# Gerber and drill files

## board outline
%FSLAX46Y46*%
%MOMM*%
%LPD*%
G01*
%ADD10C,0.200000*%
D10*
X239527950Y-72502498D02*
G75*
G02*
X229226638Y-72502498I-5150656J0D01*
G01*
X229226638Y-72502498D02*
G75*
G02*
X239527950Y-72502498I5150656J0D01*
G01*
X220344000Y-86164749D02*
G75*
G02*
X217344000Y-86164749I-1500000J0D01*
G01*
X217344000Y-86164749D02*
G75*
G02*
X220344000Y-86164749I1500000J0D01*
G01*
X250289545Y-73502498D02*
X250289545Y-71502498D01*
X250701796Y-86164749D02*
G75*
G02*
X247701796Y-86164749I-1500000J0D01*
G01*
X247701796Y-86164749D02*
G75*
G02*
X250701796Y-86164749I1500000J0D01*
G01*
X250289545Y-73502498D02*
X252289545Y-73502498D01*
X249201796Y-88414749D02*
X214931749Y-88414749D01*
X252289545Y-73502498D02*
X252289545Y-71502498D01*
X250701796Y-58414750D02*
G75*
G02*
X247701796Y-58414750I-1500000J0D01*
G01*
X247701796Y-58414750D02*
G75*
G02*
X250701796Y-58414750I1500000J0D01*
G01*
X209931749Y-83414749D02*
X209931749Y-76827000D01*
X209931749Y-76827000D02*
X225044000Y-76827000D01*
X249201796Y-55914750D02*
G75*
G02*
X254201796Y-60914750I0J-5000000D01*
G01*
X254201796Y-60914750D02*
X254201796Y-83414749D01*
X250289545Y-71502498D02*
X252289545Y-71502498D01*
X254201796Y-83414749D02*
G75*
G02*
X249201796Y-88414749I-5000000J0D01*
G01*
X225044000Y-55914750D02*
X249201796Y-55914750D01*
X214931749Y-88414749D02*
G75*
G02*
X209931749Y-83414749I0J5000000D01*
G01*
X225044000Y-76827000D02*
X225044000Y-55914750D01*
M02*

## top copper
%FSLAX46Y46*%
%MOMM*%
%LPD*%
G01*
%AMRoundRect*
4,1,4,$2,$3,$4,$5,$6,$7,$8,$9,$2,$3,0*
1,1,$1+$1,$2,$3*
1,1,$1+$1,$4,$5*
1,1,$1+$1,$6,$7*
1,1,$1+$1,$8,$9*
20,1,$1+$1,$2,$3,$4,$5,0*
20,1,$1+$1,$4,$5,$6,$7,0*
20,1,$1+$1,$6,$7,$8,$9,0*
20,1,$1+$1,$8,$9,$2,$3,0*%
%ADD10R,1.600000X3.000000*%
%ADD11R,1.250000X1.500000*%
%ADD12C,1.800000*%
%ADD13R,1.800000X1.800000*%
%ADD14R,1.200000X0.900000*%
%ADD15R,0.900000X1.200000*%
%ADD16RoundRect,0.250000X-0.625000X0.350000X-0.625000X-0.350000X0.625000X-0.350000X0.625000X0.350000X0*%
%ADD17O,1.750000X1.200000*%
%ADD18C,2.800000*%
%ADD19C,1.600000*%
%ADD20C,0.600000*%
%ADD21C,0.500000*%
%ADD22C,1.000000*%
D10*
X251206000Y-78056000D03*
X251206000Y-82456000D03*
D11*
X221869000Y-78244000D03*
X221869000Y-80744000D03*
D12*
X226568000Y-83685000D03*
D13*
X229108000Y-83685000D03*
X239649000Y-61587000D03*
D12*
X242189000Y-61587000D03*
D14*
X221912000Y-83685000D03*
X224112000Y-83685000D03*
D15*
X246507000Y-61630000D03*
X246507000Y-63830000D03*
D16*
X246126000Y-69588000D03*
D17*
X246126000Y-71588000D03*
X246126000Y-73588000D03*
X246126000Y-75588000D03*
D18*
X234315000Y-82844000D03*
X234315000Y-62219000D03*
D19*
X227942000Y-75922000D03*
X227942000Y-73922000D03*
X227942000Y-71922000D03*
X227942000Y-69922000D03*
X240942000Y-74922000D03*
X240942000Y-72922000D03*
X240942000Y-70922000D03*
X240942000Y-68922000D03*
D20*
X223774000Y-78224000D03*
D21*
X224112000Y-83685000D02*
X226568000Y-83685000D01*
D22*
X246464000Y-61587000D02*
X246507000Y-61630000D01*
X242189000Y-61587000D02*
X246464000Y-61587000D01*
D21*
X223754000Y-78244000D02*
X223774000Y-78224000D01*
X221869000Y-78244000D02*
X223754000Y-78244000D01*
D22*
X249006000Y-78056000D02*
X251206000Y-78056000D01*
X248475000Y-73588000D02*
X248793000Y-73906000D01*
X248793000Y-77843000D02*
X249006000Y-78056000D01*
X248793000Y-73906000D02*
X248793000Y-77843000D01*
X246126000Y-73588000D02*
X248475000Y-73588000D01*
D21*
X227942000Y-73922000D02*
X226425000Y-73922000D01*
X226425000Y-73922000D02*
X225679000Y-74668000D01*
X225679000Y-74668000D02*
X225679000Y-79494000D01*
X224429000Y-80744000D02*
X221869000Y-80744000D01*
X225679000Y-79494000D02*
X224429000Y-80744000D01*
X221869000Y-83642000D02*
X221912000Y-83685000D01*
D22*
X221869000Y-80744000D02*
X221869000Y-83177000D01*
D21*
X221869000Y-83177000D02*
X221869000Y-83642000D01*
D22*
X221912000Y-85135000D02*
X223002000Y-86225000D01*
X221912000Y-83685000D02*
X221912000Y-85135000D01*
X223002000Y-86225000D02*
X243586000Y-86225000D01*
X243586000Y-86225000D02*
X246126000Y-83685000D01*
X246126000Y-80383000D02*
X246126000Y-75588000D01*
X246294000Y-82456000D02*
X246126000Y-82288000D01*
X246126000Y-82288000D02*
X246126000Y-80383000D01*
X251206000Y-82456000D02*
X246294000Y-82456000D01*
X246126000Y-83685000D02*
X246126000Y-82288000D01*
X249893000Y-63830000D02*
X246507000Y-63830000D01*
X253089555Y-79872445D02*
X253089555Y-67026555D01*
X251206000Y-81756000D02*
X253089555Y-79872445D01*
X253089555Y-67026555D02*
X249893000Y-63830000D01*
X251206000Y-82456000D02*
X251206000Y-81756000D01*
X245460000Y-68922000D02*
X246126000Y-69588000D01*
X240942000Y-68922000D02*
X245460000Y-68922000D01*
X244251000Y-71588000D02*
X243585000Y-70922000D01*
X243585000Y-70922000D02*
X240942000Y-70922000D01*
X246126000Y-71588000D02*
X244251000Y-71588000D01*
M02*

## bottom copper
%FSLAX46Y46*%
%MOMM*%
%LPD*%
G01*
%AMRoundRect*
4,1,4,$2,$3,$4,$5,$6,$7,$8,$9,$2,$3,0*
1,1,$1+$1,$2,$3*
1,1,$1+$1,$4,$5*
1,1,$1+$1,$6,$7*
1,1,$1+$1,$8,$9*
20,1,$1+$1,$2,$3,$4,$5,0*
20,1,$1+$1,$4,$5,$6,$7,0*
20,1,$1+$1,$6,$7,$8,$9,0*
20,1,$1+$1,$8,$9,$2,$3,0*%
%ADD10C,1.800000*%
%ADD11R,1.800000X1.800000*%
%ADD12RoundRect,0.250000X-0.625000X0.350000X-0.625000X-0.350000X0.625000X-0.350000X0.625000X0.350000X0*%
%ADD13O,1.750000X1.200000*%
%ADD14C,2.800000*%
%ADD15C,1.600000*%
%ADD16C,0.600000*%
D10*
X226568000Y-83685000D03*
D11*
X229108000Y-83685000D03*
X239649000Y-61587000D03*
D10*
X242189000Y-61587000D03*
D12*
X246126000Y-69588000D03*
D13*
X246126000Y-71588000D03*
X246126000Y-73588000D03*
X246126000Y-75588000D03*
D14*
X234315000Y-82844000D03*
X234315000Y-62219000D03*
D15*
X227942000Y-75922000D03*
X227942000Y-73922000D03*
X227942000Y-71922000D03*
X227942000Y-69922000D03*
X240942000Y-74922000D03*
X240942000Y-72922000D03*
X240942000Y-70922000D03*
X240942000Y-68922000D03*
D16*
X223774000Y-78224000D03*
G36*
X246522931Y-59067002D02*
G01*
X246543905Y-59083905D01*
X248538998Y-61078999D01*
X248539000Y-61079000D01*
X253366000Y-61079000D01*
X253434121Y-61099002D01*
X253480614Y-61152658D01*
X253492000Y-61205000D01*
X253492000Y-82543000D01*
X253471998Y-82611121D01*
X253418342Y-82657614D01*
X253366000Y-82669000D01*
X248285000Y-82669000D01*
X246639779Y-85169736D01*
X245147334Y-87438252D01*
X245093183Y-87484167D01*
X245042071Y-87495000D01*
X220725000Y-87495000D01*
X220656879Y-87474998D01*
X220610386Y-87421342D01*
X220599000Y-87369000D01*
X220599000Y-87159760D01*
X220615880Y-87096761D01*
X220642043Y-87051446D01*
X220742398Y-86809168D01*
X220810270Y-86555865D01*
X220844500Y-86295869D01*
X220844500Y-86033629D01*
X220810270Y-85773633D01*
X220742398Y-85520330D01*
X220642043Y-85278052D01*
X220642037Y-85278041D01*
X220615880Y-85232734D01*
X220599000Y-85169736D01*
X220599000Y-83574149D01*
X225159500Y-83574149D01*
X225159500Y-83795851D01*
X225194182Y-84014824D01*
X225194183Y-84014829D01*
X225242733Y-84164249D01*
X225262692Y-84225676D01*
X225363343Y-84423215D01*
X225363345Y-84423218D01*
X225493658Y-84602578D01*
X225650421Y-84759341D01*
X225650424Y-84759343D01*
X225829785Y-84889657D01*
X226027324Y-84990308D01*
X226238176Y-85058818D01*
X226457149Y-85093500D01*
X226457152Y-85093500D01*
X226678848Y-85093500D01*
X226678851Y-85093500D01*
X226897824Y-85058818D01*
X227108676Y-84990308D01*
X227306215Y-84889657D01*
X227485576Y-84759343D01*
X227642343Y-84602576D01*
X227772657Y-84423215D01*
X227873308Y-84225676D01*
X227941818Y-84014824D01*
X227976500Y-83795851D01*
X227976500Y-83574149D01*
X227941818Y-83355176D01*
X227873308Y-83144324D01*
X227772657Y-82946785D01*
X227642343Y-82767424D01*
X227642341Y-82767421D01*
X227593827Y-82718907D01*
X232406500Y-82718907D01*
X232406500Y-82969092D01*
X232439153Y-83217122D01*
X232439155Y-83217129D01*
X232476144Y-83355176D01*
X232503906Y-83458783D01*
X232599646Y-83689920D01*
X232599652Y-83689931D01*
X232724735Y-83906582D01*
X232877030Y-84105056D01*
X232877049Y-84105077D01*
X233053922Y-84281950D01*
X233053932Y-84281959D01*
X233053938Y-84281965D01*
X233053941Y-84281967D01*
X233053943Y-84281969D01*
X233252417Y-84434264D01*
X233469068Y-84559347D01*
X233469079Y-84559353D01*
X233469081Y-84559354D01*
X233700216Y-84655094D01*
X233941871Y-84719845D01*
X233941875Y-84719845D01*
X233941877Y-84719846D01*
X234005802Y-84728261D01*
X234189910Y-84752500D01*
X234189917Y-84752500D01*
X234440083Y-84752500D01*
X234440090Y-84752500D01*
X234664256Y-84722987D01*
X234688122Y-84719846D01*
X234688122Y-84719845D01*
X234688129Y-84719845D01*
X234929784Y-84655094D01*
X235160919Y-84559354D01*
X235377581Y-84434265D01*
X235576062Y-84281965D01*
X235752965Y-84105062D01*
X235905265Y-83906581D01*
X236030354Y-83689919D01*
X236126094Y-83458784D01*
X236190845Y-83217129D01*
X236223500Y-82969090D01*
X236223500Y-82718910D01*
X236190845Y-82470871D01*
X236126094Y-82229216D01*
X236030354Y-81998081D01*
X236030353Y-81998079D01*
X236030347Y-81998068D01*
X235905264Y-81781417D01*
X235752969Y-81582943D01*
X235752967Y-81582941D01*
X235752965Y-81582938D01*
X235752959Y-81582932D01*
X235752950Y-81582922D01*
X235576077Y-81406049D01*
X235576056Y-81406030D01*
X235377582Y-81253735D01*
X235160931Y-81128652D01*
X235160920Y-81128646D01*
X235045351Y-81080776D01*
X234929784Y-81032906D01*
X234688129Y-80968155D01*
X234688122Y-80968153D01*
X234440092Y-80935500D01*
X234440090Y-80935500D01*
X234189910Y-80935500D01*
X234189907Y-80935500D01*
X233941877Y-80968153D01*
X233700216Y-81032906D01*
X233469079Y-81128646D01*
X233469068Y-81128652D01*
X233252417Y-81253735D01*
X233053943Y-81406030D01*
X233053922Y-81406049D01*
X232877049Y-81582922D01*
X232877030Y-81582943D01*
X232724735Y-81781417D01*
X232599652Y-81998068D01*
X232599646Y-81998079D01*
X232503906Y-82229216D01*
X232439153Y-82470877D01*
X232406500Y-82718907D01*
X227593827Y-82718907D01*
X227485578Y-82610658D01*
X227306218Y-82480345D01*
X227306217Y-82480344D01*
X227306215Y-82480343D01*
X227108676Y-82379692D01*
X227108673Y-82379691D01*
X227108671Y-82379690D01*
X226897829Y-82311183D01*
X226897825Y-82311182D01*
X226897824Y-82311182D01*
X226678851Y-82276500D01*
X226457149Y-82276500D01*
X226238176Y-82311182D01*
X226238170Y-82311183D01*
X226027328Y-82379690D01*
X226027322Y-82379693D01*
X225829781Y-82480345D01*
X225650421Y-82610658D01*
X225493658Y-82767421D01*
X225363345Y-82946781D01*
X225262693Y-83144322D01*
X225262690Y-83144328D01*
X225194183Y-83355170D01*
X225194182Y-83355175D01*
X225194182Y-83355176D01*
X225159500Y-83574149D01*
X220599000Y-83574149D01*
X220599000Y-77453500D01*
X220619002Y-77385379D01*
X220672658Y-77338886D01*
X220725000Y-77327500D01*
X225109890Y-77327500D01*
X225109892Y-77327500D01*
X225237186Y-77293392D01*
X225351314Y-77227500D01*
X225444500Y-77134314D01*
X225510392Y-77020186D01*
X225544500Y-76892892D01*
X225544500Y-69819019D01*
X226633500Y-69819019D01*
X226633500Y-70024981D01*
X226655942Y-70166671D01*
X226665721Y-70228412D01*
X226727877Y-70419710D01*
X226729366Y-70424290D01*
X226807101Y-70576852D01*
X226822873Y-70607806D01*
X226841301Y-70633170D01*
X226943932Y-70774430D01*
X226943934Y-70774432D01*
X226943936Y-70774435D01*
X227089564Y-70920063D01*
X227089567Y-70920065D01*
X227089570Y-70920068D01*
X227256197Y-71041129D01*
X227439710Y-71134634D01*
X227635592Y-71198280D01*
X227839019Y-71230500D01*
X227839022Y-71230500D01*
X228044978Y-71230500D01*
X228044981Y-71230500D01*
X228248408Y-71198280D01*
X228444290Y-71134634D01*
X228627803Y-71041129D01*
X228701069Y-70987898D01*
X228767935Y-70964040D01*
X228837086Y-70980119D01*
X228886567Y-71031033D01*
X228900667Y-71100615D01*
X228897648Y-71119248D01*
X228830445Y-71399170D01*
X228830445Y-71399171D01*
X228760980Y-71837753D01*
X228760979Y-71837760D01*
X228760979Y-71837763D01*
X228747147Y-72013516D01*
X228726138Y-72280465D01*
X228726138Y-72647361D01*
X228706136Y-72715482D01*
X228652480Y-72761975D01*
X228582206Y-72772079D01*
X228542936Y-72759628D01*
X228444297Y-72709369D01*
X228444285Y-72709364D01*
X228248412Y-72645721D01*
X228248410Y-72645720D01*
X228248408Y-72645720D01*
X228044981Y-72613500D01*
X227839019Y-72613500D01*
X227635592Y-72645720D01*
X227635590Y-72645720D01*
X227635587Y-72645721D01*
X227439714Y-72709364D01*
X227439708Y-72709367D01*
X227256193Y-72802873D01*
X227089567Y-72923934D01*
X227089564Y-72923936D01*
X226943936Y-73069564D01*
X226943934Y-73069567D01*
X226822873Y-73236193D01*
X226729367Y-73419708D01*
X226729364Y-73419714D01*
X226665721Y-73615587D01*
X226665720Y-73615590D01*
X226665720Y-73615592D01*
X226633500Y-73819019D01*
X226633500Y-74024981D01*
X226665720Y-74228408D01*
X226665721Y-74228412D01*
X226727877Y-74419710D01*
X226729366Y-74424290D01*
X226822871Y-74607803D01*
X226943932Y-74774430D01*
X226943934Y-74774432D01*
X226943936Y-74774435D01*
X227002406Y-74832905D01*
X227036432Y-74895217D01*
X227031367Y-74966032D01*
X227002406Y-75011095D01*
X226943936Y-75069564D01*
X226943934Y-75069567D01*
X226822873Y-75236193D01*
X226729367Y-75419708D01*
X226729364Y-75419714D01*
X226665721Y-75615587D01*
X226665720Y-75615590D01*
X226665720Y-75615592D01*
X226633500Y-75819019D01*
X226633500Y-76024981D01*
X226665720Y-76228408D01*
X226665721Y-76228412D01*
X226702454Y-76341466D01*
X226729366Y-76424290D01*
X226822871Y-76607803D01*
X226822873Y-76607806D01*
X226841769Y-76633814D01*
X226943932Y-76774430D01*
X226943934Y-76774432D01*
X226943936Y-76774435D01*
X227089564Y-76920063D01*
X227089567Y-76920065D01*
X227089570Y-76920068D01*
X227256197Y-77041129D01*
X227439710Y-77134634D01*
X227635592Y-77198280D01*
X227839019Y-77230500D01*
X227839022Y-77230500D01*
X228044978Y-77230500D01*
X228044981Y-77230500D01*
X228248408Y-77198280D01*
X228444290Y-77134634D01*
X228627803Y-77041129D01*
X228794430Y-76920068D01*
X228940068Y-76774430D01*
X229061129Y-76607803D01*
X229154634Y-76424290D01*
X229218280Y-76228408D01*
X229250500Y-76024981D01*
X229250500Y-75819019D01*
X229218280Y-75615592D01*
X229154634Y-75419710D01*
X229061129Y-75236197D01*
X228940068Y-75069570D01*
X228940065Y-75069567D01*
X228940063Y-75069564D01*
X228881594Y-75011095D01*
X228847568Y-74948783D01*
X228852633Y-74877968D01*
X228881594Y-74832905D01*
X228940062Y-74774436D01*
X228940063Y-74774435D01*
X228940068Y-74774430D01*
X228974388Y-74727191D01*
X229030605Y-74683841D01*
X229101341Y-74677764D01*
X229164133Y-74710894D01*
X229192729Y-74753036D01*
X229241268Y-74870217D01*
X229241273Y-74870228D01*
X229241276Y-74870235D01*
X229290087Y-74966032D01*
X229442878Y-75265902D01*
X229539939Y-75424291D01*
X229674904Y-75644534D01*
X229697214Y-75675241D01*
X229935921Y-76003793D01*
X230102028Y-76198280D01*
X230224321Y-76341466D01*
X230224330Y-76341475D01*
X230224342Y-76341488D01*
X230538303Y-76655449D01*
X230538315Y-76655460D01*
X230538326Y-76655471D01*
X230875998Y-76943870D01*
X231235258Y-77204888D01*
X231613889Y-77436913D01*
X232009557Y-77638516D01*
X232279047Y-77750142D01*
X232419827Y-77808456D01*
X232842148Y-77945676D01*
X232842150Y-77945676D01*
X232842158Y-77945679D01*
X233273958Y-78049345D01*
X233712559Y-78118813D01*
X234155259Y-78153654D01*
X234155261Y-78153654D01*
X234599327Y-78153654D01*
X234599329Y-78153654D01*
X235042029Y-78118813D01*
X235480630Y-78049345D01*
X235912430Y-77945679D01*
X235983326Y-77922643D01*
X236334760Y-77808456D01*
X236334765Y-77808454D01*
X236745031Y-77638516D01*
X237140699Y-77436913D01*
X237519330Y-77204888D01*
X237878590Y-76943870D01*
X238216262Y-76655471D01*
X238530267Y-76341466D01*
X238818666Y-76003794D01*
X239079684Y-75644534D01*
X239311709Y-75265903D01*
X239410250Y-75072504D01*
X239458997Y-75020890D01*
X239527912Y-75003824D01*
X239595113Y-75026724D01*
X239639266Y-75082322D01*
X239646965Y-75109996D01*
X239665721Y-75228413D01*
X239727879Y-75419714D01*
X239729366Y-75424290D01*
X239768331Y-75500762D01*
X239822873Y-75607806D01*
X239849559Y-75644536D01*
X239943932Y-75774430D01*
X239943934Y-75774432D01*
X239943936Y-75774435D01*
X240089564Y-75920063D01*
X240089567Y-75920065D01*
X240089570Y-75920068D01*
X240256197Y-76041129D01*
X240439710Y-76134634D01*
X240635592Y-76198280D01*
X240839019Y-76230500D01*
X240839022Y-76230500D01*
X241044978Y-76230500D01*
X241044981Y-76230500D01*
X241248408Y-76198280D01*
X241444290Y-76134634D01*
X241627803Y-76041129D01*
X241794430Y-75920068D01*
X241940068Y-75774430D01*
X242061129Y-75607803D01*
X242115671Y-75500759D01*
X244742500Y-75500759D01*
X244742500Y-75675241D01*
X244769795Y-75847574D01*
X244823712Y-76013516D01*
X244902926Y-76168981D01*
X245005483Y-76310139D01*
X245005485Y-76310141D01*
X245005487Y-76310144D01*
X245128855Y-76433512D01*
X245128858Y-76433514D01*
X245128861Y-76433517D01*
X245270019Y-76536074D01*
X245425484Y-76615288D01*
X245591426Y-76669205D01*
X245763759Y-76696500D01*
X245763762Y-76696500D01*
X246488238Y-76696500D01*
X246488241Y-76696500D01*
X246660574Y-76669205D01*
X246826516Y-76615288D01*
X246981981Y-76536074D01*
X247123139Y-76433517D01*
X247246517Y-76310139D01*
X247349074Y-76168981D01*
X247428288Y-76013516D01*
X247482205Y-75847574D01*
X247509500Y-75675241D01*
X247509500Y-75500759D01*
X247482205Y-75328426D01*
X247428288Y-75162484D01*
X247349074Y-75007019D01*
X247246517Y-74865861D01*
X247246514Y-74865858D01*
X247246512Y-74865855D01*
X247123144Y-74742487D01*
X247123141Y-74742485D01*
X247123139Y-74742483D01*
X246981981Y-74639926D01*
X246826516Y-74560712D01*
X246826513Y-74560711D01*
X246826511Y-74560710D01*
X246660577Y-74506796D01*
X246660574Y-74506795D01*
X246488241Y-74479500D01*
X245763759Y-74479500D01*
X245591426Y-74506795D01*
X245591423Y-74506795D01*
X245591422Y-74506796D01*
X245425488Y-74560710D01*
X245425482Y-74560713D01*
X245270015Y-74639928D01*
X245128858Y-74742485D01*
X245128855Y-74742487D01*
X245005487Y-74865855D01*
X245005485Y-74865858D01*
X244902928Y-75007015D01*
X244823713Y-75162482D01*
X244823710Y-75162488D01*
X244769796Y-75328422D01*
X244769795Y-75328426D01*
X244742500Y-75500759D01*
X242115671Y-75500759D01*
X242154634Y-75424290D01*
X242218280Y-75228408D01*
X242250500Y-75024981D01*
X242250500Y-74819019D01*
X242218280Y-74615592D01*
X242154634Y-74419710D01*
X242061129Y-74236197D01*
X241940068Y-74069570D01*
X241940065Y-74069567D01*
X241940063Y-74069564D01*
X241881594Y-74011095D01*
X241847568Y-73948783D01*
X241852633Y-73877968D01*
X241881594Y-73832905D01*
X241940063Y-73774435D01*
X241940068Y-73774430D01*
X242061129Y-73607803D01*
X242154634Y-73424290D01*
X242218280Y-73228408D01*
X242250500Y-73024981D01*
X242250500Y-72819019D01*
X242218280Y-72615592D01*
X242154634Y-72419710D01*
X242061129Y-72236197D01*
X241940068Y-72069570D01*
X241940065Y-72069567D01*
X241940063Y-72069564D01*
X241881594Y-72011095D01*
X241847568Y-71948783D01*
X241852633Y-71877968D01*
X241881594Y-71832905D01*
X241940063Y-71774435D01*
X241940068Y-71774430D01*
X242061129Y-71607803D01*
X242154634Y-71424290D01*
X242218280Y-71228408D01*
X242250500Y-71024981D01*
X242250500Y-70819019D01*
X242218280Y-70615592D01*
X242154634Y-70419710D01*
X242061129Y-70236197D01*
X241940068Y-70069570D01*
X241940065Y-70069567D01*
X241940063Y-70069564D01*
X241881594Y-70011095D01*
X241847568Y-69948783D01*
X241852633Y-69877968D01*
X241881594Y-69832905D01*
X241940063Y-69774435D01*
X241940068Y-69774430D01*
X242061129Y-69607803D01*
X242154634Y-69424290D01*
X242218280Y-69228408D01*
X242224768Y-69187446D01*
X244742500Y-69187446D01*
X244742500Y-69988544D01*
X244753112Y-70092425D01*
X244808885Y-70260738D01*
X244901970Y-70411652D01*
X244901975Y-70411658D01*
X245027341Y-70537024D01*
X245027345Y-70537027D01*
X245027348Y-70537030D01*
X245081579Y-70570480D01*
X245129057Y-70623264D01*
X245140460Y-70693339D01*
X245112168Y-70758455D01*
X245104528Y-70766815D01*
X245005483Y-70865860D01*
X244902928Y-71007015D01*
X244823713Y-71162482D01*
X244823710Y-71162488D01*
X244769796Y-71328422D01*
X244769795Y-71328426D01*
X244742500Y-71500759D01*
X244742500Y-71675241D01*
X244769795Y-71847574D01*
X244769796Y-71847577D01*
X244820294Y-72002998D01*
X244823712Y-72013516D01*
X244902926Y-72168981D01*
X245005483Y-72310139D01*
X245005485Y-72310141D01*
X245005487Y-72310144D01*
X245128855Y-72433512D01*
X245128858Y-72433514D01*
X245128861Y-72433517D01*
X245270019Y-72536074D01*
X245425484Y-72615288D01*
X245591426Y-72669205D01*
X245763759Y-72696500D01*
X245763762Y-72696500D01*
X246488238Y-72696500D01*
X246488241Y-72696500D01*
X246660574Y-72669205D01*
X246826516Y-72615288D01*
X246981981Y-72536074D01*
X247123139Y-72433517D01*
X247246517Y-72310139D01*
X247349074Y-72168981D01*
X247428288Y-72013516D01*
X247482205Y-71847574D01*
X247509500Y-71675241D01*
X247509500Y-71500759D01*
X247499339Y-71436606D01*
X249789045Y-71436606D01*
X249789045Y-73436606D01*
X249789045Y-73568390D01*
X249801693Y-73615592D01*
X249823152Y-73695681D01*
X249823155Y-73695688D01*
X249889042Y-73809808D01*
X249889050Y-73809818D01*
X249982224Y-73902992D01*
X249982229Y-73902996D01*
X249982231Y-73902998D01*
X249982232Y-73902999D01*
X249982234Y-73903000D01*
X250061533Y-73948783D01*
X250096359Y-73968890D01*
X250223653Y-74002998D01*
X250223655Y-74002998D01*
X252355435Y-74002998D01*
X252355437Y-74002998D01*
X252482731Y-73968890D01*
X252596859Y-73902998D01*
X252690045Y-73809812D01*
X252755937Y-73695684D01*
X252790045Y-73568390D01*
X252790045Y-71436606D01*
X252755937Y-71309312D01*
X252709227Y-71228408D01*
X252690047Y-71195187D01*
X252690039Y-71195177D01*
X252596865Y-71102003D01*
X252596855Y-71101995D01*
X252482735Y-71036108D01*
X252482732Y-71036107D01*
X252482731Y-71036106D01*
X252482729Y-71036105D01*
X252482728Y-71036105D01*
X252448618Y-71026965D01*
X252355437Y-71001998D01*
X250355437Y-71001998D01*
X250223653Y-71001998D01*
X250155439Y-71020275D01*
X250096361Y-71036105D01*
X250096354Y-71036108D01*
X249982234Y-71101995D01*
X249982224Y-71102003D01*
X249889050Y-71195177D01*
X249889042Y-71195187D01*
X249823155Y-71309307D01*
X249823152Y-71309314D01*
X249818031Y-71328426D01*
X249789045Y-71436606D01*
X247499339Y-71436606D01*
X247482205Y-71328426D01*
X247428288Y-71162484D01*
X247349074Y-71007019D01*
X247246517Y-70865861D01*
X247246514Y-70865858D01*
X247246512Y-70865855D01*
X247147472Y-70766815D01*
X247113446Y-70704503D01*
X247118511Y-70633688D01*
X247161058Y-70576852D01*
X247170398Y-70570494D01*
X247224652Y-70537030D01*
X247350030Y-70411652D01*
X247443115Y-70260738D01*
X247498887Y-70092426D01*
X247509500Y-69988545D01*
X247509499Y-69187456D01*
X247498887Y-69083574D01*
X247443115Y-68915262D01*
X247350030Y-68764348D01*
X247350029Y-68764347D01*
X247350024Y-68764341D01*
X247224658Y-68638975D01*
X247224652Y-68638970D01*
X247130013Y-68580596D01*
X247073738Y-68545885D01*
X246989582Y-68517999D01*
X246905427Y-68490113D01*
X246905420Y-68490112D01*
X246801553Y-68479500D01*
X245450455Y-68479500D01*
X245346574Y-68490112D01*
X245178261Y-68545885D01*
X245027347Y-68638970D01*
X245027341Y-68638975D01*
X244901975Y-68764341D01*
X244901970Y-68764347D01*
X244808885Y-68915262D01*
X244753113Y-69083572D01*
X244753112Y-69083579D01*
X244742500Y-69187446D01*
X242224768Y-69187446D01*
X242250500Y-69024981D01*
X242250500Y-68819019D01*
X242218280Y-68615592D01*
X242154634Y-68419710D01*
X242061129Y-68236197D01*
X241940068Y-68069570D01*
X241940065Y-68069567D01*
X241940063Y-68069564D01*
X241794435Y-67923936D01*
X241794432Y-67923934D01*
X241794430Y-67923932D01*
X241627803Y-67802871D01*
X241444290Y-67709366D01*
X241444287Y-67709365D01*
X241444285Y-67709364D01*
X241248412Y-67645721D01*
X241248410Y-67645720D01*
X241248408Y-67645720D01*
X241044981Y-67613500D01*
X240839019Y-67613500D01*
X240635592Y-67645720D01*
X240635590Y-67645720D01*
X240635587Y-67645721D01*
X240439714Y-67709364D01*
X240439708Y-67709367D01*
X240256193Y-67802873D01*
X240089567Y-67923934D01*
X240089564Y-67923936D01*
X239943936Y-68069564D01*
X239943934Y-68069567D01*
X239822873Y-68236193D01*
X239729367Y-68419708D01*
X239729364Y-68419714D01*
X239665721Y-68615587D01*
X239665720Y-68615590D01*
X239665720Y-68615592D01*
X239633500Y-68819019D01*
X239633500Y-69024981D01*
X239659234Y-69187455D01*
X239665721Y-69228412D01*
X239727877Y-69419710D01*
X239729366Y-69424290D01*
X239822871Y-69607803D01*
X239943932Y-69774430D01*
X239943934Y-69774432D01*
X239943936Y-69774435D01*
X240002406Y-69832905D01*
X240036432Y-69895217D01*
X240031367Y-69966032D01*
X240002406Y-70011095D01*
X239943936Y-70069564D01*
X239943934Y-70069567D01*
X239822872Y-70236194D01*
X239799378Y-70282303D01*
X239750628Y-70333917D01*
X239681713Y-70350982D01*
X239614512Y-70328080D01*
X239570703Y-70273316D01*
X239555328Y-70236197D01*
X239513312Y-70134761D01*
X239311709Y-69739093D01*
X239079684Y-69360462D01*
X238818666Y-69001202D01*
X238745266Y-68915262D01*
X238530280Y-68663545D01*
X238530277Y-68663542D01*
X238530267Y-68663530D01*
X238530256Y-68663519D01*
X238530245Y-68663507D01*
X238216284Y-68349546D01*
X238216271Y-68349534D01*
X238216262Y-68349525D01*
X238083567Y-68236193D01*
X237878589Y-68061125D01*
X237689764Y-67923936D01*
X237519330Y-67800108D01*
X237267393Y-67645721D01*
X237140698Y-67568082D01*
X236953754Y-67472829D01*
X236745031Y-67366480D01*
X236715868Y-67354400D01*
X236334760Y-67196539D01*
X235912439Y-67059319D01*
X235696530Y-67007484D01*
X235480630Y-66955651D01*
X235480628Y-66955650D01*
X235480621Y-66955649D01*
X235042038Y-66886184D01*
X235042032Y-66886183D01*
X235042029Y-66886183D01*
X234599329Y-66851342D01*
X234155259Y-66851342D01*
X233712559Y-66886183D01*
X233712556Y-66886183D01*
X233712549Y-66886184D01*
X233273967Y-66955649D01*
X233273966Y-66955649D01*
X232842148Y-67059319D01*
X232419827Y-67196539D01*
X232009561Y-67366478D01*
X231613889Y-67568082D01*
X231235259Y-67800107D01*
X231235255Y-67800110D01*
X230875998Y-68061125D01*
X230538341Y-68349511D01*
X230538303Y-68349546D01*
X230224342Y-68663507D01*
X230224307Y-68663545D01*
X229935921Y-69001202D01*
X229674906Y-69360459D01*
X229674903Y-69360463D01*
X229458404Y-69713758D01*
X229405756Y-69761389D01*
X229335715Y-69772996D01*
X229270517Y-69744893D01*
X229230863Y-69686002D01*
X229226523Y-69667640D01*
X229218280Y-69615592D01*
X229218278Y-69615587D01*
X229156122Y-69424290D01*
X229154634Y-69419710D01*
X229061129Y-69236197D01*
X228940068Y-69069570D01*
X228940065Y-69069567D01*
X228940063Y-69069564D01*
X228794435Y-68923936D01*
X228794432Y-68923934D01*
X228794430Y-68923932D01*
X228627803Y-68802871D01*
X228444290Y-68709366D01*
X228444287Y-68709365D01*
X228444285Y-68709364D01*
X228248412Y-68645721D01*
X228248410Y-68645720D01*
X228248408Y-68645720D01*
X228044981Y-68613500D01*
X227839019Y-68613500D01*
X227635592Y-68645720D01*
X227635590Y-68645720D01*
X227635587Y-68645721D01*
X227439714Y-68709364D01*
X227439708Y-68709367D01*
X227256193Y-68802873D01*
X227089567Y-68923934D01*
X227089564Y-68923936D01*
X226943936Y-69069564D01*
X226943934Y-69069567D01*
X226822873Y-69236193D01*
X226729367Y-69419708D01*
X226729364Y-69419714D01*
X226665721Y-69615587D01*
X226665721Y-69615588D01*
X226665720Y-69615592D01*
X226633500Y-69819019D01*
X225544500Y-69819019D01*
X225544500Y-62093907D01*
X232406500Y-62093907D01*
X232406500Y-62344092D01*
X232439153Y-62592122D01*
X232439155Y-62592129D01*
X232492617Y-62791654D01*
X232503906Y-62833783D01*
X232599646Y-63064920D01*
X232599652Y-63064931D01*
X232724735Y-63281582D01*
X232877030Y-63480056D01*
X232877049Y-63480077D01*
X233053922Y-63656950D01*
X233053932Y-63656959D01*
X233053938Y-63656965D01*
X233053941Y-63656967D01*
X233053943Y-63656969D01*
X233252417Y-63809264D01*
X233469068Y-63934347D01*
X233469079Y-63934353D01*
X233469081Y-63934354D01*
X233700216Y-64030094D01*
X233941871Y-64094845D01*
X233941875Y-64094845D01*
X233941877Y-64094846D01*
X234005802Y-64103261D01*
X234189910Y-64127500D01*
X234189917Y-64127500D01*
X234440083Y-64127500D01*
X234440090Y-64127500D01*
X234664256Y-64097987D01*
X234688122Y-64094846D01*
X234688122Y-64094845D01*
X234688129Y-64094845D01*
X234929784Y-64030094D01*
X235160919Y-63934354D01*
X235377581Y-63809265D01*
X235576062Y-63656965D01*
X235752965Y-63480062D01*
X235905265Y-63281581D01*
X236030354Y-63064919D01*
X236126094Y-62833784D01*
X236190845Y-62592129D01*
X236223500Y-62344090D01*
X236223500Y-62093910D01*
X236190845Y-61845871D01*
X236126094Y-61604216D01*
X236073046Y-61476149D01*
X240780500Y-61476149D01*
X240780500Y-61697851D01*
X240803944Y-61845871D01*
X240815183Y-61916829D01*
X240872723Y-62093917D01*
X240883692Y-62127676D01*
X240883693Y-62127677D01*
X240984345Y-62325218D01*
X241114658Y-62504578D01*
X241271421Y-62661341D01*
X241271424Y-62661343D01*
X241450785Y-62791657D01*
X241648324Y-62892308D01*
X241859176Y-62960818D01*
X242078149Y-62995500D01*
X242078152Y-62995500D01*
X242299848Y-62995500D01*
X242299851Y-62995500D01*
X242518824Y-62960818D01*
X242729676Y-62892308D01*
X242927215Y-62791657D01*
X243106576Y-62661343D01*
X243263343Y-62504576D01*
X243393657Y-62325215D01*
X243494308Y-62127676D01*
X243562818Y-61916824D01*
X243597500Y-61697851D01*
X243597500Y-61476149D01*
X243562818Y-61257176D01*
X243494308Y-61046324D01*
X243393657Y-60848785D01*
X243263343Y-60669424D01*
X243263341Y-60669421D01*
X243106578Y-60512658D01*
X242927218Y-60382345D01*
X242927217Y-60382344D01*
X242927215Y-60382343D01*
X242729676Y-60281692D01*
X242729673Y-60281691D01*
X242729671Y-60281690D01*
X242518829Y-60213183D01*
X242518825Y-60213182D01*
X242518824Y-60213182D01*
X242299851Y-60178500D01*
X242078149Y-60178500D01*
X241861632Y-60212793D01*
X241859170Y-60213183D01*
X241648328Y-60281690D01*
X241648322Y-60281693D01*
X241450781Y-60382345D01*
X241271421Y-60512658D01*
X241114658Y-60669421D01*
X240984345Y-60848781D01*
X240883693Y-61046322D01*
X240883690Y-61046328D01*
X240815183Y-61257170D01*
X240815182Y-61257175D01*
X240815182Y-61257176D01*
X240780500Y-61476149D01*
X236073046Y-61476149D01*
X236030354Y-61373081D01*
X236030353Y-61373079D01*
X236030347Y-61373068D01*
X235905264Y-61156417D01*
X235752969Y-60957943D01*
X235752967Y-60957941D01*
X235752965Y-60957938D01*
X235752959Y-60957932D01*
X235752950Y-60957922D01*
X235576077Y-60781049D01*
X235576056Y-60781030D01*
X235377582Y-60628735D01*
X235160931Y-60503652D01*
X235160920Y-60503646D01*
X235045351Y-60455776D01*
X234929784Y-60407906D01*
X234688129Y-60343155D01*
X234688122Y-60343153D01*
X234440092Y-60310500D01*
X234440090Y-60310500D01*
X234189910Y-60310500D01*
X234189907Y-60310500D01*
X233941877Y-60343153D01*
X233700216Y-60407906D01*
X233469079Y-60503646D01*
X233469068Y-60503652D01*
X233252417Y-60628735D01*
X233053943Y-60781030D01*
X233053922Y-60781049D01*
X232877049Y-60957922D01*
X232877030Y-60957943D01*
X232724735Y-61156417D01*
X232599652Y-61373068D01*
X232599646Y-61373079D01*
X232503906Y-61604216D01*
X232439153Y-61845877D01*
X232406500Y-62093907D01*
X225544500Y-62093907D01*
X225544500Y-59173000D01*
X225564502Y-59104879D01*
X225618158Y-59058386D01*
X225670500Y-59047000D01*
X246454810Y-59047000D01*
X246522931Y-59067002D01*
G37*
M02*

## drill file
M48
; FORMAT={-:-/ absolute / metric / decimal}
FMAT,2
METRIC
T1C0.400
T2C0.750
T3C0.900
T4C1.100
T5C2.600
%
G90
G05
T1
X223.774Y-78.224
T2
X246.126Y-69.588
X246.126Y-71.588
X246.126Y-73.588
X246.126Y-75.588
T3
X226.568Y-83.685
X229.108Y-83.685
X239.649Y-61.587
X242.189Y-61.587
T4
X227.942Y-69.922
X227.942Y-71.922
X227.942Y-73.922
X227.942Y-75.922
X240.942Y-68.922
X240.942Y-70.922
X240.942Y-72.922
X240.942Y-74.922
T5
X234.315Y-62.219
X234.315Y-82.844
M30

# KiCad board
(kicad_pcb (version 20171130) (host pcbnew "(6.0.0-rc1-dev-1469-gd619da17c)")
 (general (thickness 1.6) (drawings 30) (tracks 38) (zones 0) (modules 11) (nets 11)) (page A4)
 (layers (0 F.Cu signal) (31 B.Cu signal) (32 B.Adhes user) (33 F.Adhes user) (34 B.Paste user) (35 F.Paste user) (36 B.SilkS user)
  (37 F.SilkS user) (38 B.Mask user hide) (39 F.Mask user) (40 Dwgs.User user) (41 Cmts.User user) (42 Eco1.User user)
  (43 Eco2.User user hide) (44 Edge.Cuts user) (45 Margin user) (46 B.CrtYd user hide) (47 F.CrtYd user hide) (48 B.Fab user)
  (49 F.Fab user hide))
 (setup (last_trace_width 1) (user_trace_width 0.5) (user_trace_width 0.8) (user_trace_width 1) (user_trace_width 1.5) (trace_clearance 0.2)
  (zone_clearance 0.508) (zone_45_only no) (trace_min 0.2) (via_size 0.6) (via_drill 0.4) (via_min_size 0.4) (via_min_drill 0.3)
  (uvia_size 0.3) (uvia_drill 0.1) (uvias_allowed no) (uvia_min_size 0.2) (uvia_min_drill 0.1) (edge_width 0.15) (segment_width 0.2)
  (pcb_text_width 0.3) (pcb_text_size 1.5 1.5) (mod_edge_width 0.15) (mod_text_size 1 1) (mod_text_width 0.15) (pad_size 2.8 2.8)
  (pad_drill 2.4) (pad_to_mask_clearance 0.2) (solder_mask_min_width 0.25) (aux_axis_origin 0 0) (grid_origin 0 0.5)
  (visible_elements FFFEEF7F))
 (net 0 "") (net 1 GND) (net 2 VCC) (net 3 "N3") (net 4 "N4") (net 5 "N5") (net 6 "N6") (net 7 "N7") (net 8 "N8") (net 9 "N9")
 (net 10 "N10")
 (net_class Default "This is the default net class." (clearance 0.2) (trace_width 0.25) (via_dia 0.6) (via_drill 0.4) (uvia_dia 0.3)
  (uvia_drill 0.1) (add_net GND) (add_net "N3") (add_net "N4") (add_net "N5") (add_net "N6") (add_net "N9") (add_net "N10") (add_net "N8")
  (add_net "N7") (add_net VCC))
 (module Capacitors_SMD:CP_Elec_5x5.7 (layer F.Cu) (at 251.206 80.256 90)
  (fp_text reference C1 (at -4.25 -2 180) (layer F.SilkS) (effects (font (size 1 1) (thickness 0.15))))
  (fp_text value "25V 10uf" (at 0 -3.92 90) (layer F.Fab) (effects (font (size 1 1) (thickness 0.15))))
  (pad 2 smd rect (at 2.2 0 270) (size 3 1.6) (layers F.Cu F.Paste F.Mask) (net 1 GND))
  (pad 1 smd rect (at -2.2 0 270) (size 3 1.6) (layers F.Cu F.Paste F.Mask) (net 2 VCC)))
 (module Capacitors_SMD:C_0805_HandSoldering (layer F.Cu) (at 221.869 79.494 90)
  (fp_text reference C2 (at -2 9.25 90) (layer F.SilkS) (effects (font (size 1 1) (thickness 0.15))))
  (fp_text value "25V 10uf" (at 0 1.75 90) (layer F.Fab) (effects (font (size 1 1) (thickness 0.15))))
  (pad 2 smd rect (at 1.25 0 90) (size 1.5 1.25) (layers F.Cu F.Paste F.Mask) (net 1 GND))
  (pad 1 smd rect (at -1.25 0 90) (size 1.5 1.25) (layers F.Cu F.Paste F.Mask) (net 2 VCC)))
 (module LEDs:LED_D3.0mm (layer F.Cu) (at 229.108 83.685 180)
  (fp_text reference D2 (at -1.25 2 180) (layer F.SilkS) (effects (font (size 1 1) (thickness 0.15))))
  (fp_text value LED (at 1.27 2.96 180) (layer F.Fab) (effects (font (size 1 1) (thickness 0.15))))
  (pad 2 thru_hole circle (at 2.54 0 180) (size 1.8 1.8) (drill 0.9) (layers *.Cu *.Mask) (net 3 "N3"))
  (pad 1 thru_hole rect (at 0 0 180) (size 1.8 1.8) (drill 0.9) (layers *.Cu *.Mask) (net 1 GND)))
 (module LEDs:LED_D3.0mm (layer F.Cu) (at 239.649 61.587)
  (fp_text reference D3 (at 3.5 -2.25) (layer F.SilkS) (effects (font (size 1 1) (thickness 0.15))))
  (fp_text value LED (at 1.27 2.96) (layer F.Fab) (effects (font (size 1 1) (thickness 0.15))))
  (pad 1 thru_hole rect (at 0 0) (size 1.8 1.8) (drill 0.9) (layers *.Cu *.Mask) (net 1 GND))
  (pad 2 thru_hole circle (at 2.54 0) (size 1.8 1.8) (drill 0.9) (layers *.Cu *.Mask) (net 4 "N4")))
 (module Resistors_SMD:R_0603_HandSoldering (layer F.Cu) (at 223.012 83.685 180)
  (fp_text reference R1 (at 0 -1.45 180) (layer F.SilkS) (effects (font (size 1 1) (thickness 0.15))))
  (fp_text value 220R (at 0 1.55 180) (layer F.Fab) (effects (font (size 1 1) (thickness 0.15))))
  (pad 2 smd rect (at 1.1 0 180) (size 1.2 0.9) (layers F.Cu F.Paste F.Mask) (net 2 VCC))
  (pad 1 smd rect (at -1.1 0 180) (size 1.2 0.9) (layers F.Cu F.Paste F.Mask) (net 3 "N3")))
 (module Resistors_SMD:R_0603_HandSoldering (layer F.Cu) (at 246.507 62.73 270)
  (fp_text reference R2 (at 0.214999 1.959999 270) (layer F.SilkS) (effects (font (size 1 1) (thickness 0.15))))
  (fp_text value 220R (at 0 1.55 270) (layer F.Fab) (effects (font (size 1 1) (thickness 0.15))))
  (pad 1 smd rect (at -1.1 0 270) (size 1.2 0.9) (layers F.Cu F.Paste F.Mask) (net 4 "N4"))
  (pad 2 smd rect (at 1.1 0 270) (size 1.2 0.9) (layers F.Cu F.Paste F.Mask) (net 2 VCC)))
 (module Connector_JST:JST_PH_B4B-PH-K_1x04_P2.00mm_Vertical (layer F.Cu) (at 246.126 69.588 270)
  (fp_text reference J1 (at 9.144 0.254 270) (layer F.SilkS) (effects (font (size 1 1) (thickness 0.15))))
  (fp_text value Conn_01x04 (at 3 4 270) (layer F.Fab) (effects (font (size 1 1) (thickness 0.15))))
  (pad 1 thru_hole roundrect (at 0 0 270) (size 1.2 1.75) (drill 0.75) (layers *.Cu *.Mask) (roundrect_rratio 0.208333) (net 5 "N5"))
  (pad 2 thru_hole oval (at 2 0 270) (size 1.2 1.75) (drill 0.75) (layers *.Cu *.Mask) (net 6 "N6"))
  (pad 3 thru_hole oval (at 4 0 270) (size 1.2 1.75) (drill 0.75) (layers *.Cu *.Mask) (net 1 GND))
  (pad 4 thru_hole oval (at 6 0 270) (size 1.2 1.75) (drill 0.75) (layers *.Cu *.Mask) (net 2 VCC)))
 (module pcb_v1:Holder (layer F.Cu) (at 234.315 69.969)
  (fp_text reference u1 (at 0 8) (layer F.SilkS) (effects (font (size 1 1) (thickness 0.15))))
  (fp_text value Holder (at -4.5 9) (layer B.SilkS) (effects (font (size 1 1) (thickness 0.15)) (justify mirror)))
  (pad 1 thru_hole circle (at 0 12.875) (size 2.8 2.8) (drill 2.6) (layers *.Cu *.Mask))
  (pad 2 thru_hole circle (at 0 -7.75) (size 2.8 2.8) (drill 2.6) (layers *.Cu *.Mask)))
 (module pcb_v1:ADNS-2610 (layer F.Cu) (at 234.442 74.922)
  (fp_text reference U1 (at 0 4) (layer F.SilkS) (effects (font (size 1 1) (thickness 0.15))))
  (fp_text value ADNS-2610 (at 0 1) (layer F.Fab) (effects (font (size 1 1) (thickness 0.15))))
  (pad 8 thru_hole circle (at -6.5 1) (size 1.6 1.6) (drill 1.1) (layers *.Cu *.Mask) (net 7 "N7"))
  (pad 7 thru_hole circle (at -6.5 -1) (size 1.6 1.6) (drill 1.1) (layers *.Cu *.Mask) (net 2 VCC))
  (pad 6 thru_hole circle (at -6.5 -3) (size 1.6 1.6) (drill 1.1) (layers *.Cu *.Mask) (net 1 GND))
  (pad 5 thru_hole circle (at -6.5 -5) (size 1.6 1.6) (drill 1.1) (layers *.Cu *.Mask) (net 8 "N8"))
  (pad 1 thru_hole circle (at 6.5 0) (size 1.6 1.6) (drill 1.1) (layers *.Cu *.Mask) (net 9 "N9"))
  (pad 2 thru_hole circle (at 6.5 -2) (size 1.6 1.6) (drill 1.1) (layers *.Cu *.Mask) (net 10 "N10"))
  (pad 3 thru_hole circle (at 6.5 -4) (size 1.6 1.6) (drill 1.1) (layers *.Cu *.Mask) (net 6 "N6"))
  (pad 4 thru_hole circle (at 6.5 -6) (size 1.6 1.6) (drill 1.1) (layers *.Cu *.Mask) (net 5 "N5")))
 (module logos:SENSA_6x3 (layer F.Cu) (at 213.233 80.256)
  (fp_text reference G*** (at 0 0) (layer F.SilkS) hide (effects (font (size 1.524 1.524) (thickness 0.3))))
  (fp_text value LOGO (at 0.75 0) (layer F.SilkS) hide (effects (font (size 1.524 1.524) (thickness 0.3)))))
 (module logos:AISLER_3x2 (layer F.Cu) (at 218.567 80.383)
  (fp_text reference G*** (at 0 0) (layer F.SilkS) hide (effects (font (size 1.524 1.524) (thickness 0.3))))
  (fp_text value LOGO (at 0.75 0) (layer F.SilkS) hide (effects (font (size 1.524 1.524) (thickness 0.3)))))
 (gr_circle (center 234.377294 72.502498) (end 239.522 72.255) (layer Edge.Cuts) (width 0.2))
 (gr_circle (center 218.844 86.164749) (end 220.344 86.164749) (layer Edge.Cuts) (width 0.2))
 (gr_line (start 250.289545 73.502498) (end 250.289545 71.502498) (layer Edge.Cuts) (width 0.2))
 (gr_circle (center 249.201796 86.164749) (end 250.701796 86.164749) (layer Edge.Cuts) (width 0.2))
 (gr_line (start 250.289545 73.502498) (end 252.289545 73.502498) (layer Edge.Cuts) (width 0.2))
 (gr_line (start 249.201796 88.414749) (end 214.931749 88.414749) (layer Edge.Cuts) (width 0.2))
 (gr_line (start 252.289545 73.502498) (end 252.289545 71.502498) (layer Edge.Cuts) (width 0.2))
 (gr_circle (center 249.201796 58.41475) (end 250.701796 58.41475) (layer Edge.Cuts) (width 0.2))
 (gr_line (start 209.931749 83.414749) (end 209.931749 76.827) (layer Edge.Cuts) (width 0.2))
 (gr_line (start 209.931749 76.827) (end 225.044 76.827) (layer Edge.Cuts) (width 0.2))
 (gr_arc (start 249.201796 60.91475) (end 254.201796 60.91475) (angle -90) (layer Edge.Cuts) (width 0.2))
 (gr_line (start 254.201796 60.91475) (end 254.201796 83.414749) (layer Edge.Cuts) (width 0.2))
 (gr_line (start 250.289545 71.502498) (end 252.289545 71.502498) (layer Edge.Cuts) (width 0.2))
 (gr_arc (start 249.201796 83.414749) (end 249.201796 88.414749) (angle -90) (layer Edge.Cuts) (width 0.2))
 (gr_line (start 225.044 55.91475) (end 249.201796 55.91475) (layer Edge.Cuts) (width 0.2))
 (gr_arc (start 214.931749 83.414749) (end 209.931749 83.414749) (angle -90) (layer Edge.Cuts) (width 0.2))
 (gr_line (start 225.044 76.827) (end 225.044 55.91475) (layer Edge.Cuts) (width 0.2))
 (segment (start 224.112 83.685) (end 226.568 83.685) (width 0.5) (layer F.Cu) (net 3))
 (segment (start 246.464 61.587) (end 246.507 61.63) (width 1) (layer F.Cu) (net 4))
 (segment (start 242.189 61.587) (end 246.464 61.587) (width 1) (layer F.Cu) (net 4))
 (segment (start 223.754 78.244) (end 223.774 78.224) (width 0.5) (layer F.Cu) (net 1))
 (via (at 223.774 78.224) (size 0.6) (drill 0.4) (layers F.Cu B.Cu) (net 1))
 (segment (start 221.869 78.244) (end 223.754 78.244) (width 0.5) (layer F.Cu) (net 1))
 (segment (start 249.006 78.056) (end 251.206 78.056) (width 1) (layer F.Cu) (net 1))
 (segment (start 248.475 73.588) (end 248.793 73.906) (width 1) (layer F.Cu) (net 1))
 (segment (start 248.793 77.843) (end 249.006 78.056) (width 1) (layer F.Cu) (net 1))
 (segment (start 248.793 73.906) (end 248.793 77.843) (width 1) (layer F.Cu) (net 1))
 (segment (start 246.126 73.588) (end 248.475 73.588) (width 1) (layer F.Cu) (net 1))
 (segment (start 227.942 73.922) (end 226.425 73.922) (width 0.5) (layer F.Cu) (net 2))
 (segment (start 226.425 73.922) (end 225.679 74.668) (width 0.5) (layer F.Cu) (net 2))
 (segment (start 225.679 74.668) (end 225.679 79.494) (width 0.5) (layer F.Cu) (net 2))
 (segment (start 224.429 80.744) (end 221.869 80.744) (width 0.5) (layer F.Cu) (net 2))
 (segment (start 225.679 79.494) (end 224.429 80.744) (width 0.5) (layer F.Cu) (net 2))
 (segment (start 221.869 83.642) (end 221.912 83.685) (width 0.5) (layer F.Cu) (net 2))
 (segment (start 221.869 80.744) (end 221.869 83.177) (width 1) (layer F.Cu) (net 2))
 (segment (start 221.869 83.177) (end 221.869 83.642) (width 0.5) (layer F.Cu) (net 2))
 (segment (start 221.912 85.135) (end 223.002 86.225) (width 1) (layer F.Cu) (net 2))
 (segment (start 221.912 83.685) (end 221.912 85.135) (width 1) (layer F.Cu) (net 2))
 (segment (start 223.002 86.225) (end 243.586 86.225) (width 1) (layer F.Cu) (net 2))
 (segment (start 243.586 86.225) (end 246.126 83.685) (width 1) (layer F.Cu) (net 2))
 (segment (start 246.126 80.383) (end 246.126 75.588) (width 1) (layer F.Cu) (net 2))
 (segment (start 246.294 82.456) (end 246.126 82.288) (width 1) (layer F.Cu) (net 2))
 (segment (start 246.126 82.288) (end 246.126 80.383) (width 1) (layer F.Cu) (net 2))
 (segment (start 251.206 82.456) (end 246.294 82.456) (width 1) (layer F.Cu) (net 2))
 (segment (start 246.126 83.685) (end 246.126 82.288) (width 1) (layer F.Cu) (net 2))
 (segment (start 249.893 63.83) (end 246.507 63.83) (width 1) (layer F.Cu) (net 2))
 (segment (start 253.089555 79.872445) (end 253.089555 67.026555) (width 1) (layer F.Cu) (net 2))
 (segment (start 251.206 81.756) (end 253.089555 79.872445) (width 1) (layer F.Cu) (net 2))
 (segment (start 253.089555 67.026555) (end 249.893 63.83) (width 1) (layer F.Cu) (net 2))
 (segment (start 251.206 82.456) (end 251.206 81.756) (width 1) (layer F.Cu) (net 2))
 (segment (start 245.46 68.922) (end 246.126 69.588) (width 1) (layer F.Cu) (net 5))
 (segment (start 240.942 68.922) (end 245.46 68.922) (width 1) (layer F.Cu) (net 5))
 (segment (start 244.251 71.588) (end 243.585 70.922) (width 1) (layer F.Cu) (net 6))
 (segment (start 243.585 70.922) (end 240.942 70.922) (width 1) (layer F.Cu) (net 6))
 (segment (start 246.126 71.588) (end 244.251 71.588) (width 1) (layer F.Cu) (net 6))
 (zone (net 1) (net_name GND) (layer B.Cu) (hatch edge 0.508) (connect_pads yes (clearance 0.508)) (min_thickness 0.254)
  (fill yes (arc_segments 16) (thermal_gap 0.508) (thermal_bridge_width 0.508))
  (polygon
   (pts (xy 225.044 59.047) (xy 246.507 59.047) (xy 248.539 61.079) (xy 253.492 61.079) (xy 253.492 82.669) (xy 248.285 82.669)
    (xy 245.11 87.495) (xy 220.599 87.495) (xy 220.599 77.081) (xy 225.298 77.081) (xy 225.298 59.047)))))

